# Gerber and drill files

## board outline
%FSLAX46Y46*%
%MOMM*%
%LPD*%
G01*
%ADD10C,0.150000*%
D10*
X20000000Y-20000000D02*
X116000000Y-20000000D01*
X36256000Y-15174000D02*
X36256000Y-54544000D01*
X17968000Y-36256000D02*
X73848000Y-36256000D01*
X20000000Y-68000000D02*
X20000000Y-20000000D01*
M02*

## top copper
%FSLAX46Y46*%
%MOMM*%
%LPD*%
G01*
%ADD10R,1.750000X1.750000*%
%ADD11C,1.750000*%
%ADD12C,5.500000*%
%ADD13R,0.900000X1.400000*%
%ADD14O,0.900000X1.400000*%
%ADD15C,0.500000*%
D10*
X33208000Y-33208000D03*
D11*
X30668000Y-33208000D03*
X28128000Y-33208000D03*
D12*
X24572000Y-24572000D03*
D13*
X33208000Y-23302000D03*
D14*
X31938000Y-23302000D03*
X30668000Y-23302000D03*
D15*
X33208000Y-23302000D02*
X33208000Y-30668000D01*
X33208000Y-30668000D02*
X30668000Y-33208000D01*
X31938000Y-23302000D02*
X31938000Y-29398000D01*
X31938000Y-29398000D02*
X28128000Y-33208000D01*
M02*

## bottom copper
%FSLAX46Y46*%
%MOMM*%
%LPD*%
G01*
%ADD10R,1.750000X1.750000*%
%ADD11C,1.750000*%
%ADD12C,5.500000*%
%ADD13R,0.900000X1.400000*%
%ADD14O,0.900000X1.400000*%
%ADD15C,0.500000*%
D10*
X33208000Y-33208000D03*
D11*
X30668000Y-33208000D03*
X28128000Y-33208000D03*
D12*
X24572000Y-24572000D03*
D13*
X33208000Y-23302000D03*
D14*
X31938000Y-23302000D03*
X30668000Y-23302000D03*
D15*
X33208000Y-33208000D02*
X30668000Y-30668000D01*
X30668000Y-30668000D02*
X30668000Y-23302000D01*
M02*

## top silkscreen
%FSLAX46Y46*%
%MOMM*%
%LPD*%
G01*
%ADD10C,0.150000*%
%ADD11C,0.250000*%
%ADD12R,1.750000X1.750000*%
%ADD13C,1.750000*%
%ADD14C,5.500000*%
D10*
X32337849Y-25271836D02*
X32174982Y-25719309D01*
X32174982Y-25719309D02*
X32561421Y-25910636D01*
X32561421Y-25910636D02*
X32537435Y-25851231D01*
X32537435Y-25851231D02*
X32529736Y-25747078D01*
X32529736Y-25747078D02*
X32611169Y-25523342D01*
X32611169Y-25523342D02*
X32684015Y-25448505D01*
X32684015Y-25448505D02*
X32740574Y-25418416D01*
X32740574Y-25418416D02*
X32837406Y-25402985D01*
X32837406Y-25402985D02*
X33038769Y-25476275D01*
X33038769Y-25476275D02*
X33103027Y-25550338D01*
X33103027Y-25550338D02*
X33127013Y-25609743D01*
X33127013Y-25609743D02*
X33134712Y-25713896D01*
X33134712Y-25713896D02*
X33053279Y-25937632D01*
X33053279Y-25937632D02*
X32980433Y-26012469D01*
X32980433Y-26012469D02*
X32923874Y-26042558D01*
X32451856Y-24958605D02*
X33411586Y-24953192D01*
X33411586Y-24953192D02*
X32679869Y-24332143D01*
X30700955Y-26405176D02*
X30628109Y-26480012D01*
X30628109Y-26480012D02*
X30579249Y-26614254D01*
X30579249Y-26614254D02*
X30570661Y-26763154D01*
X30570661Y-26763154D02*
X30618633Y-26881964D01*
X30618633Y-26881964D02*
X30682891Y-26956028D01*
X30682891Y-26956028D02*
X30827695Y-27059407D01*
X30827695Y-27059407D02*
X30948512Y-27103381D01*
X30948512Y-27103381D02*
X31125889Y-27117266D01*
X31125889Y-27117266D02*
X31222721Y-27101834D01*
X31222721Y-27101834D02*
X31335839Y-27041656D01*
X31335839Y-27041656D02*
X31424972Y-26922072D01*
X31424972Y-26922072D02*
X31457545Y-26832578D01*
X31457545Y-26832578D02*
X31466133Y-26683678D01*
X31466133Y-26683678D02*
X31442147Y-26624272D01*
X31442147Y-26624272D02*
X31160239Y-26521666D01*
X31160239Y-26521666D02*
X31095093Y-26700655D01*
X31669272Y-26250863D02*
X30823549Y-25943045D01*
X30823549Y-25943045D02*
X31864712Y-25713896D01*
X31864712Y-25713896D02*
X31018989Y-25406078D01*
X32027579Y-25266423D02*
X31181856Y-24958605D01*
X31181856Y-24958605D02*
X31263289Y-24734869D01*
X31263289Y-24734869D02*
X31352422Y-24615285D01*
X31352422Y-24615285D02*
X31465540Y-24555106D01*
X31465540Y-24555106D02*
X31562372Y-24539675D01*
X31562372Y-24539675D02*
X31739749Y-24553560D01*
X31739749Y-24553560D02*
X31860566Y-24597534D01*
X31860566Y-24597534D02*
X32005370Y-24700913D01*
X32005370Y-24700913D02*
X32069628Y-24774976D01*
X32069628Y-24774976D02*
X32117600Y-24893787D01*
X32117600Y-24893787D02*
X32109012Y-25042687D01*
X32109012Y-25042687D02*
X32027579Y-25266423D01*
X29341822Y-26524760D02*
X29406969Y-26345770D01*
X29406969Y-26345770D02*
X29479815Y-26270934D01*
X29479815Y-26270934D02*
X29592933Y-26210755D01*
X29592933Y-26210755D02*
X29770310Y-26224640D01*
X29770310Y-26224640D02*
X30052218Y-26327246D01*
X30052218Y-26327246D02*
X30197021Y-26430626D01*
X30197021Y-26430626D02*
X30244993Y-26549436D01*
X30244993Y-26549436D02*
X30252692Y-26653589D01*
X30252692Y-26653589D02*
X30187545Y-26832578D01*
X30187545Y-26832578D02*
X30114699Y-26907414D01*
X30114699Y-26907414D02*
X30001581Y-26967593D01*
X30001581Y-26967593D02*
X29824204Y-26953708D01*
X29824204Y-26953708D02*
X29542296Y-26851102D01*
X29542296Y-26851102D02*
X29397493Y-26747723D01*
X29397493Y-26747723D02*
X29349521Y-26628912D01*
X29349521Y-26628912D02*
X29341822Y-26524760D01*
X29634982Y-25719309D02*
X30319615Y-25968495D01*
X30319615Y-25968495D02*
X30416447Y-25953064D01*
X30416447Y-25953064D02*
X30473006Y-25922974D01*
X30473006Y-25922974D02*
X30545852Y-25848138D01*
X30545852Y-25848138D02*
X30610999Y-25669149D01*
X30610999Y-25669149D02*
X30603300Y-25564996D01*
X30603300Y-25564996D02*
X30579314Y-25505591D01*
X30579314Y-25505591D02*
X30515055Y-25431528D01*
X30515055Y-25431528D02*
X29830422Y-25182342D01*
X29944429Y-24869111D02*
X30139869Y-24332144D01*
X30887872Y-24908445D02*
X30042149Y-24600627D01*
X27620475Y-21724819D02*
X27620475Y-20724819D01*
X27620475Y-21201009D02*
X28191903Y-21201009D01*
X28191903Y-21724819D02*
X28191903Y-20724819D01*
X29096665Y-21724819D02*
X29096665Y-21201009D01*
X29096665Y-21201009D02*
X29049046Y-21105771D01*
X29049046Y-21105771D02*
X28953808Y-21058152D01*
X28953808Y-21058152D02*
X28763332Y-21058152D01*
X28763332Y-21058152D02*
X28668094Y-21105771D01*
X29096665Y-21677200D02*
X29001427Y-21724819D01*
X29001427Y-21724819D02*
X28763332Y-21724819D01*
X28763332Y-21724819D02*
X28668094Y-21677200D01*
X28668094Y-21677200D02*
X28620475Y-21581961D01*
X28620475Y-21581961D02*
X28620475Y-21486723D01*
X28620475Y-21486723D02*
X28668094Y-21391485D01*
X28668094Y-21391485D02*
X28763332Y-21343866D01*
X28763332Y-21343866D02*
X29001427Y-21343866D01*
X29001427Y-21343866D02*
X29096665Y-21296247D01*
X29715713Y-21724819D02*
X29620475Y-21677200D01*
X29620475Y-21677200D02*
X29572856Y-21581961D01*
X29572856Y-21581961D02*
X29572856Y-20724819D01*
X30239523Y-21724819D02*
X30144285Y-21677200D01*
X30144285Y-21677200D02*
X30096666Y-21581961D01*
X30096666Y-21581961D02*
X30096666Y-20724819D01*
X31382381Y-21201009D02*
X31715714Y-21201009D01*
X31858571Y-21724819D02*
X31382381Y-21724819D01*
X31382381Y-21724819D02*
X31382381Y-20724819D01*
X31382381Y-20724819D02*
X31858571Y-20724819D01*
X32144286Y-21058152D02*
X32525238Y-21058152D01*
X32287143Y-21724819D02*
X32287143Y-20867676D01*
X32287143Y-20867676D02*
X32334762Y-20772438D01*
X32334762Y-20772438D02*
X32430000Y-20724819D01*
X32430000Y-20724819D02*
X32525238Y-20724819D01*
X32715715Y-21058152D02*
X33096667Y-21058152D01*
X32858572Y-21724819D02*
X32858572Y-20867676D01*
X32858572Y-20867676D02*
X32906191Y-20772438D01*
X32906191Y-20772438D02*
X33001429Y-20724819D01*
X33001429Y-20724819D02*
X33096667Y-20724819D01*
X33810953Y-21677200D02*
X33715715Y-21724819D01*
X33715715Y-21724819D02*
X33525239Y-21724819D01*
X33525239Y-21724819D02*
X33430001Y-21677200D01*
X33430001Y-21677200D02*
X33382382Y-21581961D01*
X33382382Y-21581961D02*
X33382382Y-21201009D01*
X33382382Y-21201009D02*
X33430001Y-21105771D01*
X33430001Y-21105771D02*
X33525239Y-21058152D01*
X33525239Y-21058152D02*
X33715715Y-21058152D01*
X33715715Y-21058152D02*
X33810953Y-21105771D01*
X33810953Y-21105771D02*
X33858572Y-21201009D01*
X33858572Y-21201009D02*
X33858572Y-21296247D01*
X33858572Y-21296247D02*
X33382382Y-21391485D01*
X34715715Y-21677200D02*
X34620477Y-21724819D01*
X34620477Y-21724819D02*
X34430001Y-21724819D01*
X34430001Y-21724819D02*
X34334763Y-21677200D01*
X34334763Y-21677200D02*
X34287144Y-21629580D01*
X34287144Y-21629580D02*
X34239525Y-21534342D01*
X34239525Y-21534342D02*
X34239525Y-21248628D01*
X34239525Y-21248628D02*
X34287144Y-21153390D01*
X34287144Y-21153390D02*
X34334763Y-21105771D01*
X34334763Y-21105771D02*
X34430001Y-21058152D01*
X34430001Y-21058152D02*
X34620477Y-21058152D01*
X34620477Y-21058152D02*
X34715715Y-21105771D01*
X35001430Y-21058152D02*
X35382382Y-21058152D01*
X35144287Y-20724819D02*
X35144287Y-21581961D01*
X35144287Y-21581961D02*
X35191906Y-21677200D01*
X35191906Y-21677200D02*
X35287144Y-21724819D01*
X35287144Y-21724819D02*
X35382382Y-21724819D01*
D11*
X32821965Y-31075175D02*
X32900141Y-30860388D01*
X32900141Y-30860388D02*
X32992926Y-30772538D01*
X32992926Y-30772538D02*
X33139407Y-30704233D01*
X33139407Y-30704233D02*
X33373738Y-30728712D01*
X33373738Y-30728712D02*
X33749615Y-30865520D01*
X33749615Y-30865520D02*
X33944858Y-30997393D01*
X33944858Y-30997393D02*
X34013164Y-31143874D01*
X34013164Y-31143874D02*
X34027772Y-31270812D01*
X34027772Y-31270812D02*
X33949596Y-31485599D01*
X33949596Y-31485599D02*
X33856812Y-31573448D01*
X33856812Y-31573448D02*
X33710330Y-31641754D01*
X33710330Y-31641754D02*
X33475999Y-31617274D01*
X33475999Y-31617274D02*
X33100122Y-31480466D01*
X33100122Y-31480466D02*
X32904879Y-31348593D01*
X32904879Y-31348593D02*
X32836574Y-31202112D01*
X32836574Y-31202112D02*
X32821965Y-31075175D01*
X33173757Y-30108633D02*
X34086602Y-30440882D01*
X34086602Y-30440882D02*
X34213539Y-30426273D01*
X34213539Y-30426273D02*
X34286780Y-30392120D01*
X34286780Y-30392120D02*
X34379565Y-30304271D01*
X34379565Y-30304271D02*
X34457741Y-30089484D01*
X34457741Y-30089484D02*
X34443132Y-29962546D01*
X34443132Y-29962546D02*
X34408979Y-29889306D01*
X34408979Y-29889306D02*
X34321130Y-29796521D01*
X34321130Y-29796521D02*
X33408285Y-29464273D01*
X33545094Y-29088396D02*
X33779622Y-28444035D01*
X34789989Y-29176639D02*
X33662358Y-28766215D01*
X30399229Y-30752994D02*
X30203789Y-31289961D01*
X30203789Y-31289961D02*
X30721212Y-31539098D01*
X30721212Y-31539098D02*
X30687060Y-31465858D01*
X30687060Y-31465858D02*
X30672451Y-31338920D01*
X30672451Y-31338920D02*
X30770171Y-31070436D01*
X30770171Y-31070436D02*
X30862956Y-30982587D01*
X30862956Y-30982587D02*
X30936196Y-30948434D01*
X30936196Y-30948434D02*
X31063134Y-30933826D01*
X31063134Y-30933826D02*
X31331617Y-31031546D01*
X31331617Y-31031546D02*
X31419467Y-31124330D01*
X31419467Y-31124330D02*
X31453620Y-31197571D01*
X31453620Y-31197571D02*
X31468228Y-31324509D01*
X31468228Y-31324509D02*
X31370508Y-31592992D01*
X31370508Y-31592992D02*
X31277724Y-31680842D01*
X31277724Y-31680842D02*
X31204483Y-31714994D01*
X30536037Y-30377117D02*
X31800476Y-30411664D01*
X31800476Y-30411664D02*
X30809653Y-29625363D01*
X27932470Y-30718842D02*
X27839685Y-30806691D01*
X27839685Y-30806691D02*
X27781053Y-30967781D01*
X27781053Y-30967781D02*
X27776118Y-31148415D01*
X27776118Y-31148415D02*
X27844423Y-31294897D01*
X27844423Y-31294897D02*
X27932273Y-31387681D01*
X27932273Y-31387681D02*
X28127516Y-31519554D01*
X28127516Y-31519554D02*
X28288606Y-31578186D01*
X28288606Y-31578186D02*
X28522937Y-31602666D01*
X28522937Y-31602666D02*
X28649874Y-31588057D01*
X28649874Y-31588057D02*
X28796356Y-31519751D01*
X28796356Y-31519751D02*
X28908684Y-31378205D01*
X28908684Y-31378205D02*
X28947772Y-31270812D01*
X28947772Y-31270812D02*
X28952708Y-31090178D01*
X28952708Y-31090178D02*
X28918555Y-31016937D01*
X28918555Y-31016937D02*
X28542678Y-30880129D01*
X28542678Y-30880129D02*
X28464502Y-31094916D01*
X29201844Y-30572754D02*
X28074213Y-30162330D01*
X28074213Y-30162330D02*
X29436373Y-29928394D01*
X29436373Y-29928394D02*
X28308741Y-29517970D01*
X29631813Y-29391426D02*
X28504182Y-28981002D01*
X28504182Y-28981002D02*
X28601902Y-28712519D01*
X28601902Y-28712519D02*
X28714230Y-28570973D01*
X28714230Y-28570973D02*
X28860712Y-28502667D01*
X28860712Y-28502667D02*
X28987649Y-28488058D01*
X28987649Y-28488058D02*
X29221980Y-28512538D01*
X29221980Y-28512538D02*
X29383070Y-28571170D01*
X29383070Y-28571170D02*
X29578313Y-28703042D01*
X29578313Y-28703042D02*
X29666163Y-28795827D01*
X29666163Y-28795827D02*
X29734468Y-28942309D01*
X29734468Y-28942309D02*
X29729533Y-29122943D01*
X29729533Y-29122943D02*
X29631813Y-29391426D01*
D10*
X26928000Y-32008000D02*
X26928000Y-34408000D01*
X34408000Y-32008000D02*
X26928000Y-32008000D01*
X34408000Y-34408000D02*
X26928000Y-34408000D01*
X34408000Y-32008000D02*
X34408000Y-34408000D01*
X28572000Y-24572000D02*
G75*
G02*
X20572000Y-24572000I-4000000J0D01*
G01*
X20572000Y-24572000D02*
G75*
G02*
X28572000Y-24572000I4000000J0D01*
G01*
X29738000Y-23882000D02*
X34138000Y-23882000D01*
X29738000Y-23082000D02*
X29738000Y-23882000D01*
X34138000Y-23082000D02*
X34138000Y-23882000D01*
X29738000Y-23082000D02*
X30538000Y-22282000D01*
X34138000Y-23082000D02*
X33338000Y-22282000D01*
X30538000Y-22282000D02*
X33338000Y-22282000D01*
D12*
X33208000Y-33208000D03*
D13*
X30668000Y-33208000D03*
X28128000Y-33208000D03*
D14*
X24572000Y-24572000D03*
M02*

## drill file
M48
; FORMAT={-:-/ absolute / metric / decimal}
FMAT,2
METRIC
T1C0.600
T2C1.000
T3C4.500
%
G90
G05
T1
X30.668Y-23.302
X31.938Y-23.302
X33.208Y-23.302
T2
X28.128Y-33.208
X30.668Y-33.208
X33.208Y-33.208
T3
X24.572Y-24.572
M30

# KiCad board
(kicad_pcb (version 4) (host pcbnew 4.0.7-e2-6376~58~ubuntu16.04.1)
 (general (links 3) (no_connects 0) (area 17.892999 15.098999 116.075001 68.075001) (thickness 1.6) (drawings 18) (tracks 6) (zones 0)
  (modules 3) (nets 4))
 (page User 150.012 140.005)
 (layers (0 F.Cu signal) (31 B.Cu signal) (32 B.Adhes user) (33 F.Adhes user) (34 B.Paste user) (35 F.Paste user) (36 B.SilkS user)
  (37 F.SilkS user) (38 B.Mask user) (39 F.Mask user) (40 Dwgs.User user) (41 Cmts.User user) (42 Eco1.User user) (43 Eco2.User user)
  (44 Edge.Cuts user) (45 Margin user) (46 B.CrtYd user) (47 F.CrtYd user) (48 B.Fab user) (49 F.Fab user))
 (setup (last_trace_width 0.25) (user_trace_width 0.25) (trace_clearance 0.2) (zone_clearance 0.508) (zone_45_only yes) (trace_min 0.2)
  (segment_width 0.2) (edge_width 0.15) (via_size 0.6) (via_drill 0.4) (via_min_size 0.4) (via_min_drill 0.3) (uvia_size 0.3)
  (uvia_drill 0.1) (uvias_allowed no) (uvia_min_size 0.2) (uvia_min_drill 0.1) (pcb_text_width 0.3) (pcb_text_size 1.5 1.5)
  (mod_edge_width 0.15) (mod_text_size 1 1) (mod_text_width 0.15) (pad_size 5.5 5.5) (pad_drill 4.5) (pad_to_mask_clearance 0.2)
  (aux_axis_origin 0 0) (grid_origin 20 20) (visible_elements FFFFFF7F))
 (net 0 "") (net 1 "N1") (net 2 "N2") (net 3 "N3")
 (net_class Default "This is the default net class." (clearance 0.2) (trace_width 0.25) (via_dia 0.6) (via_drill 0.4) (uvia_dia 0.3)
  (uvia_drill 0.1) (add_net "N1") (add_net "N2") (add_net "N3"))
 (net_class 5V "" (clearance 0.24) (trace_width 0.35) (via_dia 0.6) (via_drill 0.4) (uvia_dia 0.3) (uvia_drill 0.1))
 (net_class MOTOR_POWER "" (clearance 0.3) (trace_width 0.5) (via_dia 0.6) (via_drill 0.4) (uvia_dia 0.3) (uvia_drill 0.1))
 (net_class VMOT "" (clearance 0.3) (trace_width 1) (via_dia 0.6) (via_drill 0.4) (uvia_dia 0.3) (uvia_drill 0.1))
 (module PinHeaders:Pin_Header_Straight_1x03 (layer F.Cu) (at 33.208 33.208 270)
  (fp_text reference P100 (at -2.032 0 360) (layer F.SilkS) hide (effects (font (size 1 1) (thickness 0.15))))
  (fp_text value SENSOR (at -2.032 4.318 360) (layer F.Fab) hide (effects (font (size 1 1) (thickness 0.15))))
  (fp_line (start -1.2 6.28) (end 1.2 6.28) (layer F.SilkS) (width 0.15))
  (fp_line (start -1.2 -1.2) (end -1.2 6.28) (layer F.SilkS) (width 0.15))
  (fp_line (start 1.2 -1.2) (end 1.2 6.28) (layer F.SilkS) (width 0.15))
  (fp_line (start -1.2 -1.2) (end 1.2 -1.2) (layer F.SilkS) (width 0.15))
  (pad 1 thru_hole rect (at 0 0 270) (size 1.75 1.75) (drill 1) (layers *.Cu *.Mask F.SilkS) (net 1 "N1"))
  (pad 2 thru_hole circle (at 0 2.54 270) (size 1.75 1.75) (drill 1) (layers *.Cu *.Mask F.SilkS) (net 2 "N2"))
  (pad 3 thru_hole circle (at 0 5.08 270) (size 1.75 1.75) (drill 1) (layers *.Cu *.Mask F.SilkS) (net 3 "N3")))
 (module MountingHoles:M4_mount (layer F.Cu) (at 24.572 24.572)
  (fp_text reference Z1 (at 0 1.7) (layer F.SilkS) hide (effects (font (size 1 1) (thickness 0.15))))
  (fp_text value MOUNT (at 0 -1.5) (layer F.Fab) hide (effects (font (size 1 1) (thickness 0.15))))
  (fp_circle (center 0 0) (end 4 0) (layer F.SilkS) (width 0.15))
  (pad 1 thru_hole circle (at 0 0) (size 5.5 5.5) (drill 4.5) (layers *.Cu *.Mask F.SilkS) (clearance 1.5)))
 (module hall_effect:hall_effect (layer B.Cu) (at 31.938 23.302 180)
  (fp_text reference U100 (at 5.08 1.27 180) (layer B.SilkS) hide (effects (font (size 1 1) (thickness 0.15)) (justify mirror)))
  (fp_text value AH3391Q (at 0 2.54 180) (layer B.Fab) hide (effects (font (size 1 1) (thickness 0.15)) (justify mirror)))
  (fp_line (start 2.2 -0.58) (end -2.2 -0.58) (layer F.SilkS) (width 0.15))
  (fp_line (start 2.2 0.22) (end 2.2 -0.58) (layer F.SilkS) (width 0.15))
  (fp_line (start -2.2 0.22) (end -2.2 -0.58) (layer F.SilkS) (width 0.15))
  (fp_line (start 2.2 0.22) (end 1.4 1.02) (layer F.SilkS) (width 0.15))
  (fp_line (start -2.2 0.22) (end -1.4 1.02) (layer F.SilkS) (width 0.15))
  (fp_line (start 1.4 1.02) (end -1.4 1.02) (layer F.SilkS) (width 0.15))
  (pad 1 thru_hole rect (at -1.27 0 180) (size 0.9 1.4) (drill 0.6) (layers *.Cu *.Mask) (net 2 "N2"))
  (pad 2 thru_hole oval (at 0 0 180) (size 0.9 1.4) (drill 0.6) (layers *.Cu *.Mask) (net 3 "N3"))
  (pad 3 thru_hole oval (at 1.27 0 180) (size 0.9 1.4) (drill 0.6) (layers *.Cu *.Mask) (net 1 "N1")))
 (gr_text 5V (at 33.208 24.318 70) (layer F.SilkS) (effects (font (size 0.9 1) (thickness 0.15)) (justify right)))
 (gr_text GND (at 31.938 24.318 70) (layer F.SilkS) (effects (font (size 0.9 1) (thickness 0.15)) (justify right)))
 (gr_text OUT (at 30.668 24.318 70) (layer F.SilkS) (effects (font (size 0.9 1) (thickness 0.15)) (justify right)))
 (gr_line (start 20 20) (end 116 20) (angle 90) (layer Edge.Cuts) (width 0.15))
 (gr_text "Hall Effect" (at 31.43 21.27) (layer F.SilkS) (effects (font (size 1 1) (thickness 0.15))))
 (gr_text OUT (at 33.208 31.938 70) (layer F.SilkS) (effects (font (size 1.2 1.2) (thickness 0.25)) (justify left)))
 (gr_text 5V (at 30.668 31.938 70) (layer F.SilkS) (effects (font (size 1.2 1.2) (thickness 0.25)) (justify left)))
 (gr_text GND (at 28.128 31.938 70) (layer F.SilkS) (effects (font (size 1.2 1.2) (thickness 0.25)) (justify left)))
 (gr_line (start 36.256 15.174) (end 36.256 54.544) (angle 90) (layer Edge.Cuts) (width 0.15))
 (gr_line (start 17.968 36.256) (end 73.848 36.256) (angle 90) (layer Edge.Cuts) (width 0.15))
 (gr_line (start 20 68) (end 20 20) (angle 90) (layer Edge.Cuts) (width 0.15))
 (segment (start 33.208 33.208) (end 30.668 30.668) (width 0.5) (layer B.Cu) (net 1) (status 10))
 (segment (start 30.668 30.668) (end 30.668 23.302) (width 0.5) (layer B.Cu) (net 1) (status 20))
 (segment (start 33.208 23.302) (end 33.208 30.668) (width 0.5) (layer F.Cu) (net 2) (status 10))
 (segment (start 33.208 30.668) (end 30.668 33.208) (width 0.5) (layer F.Cu) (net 2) (status 20))
 (segment (start 31.938 23.302) (end 31.938 29.398) (width 0.5) (layer F.Cu) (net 3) (status 10))
 (segment (start 31.938 29.398) (end 28.128 33.208) (width 0.5) (layer F.Cu) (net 3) (status 20)))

